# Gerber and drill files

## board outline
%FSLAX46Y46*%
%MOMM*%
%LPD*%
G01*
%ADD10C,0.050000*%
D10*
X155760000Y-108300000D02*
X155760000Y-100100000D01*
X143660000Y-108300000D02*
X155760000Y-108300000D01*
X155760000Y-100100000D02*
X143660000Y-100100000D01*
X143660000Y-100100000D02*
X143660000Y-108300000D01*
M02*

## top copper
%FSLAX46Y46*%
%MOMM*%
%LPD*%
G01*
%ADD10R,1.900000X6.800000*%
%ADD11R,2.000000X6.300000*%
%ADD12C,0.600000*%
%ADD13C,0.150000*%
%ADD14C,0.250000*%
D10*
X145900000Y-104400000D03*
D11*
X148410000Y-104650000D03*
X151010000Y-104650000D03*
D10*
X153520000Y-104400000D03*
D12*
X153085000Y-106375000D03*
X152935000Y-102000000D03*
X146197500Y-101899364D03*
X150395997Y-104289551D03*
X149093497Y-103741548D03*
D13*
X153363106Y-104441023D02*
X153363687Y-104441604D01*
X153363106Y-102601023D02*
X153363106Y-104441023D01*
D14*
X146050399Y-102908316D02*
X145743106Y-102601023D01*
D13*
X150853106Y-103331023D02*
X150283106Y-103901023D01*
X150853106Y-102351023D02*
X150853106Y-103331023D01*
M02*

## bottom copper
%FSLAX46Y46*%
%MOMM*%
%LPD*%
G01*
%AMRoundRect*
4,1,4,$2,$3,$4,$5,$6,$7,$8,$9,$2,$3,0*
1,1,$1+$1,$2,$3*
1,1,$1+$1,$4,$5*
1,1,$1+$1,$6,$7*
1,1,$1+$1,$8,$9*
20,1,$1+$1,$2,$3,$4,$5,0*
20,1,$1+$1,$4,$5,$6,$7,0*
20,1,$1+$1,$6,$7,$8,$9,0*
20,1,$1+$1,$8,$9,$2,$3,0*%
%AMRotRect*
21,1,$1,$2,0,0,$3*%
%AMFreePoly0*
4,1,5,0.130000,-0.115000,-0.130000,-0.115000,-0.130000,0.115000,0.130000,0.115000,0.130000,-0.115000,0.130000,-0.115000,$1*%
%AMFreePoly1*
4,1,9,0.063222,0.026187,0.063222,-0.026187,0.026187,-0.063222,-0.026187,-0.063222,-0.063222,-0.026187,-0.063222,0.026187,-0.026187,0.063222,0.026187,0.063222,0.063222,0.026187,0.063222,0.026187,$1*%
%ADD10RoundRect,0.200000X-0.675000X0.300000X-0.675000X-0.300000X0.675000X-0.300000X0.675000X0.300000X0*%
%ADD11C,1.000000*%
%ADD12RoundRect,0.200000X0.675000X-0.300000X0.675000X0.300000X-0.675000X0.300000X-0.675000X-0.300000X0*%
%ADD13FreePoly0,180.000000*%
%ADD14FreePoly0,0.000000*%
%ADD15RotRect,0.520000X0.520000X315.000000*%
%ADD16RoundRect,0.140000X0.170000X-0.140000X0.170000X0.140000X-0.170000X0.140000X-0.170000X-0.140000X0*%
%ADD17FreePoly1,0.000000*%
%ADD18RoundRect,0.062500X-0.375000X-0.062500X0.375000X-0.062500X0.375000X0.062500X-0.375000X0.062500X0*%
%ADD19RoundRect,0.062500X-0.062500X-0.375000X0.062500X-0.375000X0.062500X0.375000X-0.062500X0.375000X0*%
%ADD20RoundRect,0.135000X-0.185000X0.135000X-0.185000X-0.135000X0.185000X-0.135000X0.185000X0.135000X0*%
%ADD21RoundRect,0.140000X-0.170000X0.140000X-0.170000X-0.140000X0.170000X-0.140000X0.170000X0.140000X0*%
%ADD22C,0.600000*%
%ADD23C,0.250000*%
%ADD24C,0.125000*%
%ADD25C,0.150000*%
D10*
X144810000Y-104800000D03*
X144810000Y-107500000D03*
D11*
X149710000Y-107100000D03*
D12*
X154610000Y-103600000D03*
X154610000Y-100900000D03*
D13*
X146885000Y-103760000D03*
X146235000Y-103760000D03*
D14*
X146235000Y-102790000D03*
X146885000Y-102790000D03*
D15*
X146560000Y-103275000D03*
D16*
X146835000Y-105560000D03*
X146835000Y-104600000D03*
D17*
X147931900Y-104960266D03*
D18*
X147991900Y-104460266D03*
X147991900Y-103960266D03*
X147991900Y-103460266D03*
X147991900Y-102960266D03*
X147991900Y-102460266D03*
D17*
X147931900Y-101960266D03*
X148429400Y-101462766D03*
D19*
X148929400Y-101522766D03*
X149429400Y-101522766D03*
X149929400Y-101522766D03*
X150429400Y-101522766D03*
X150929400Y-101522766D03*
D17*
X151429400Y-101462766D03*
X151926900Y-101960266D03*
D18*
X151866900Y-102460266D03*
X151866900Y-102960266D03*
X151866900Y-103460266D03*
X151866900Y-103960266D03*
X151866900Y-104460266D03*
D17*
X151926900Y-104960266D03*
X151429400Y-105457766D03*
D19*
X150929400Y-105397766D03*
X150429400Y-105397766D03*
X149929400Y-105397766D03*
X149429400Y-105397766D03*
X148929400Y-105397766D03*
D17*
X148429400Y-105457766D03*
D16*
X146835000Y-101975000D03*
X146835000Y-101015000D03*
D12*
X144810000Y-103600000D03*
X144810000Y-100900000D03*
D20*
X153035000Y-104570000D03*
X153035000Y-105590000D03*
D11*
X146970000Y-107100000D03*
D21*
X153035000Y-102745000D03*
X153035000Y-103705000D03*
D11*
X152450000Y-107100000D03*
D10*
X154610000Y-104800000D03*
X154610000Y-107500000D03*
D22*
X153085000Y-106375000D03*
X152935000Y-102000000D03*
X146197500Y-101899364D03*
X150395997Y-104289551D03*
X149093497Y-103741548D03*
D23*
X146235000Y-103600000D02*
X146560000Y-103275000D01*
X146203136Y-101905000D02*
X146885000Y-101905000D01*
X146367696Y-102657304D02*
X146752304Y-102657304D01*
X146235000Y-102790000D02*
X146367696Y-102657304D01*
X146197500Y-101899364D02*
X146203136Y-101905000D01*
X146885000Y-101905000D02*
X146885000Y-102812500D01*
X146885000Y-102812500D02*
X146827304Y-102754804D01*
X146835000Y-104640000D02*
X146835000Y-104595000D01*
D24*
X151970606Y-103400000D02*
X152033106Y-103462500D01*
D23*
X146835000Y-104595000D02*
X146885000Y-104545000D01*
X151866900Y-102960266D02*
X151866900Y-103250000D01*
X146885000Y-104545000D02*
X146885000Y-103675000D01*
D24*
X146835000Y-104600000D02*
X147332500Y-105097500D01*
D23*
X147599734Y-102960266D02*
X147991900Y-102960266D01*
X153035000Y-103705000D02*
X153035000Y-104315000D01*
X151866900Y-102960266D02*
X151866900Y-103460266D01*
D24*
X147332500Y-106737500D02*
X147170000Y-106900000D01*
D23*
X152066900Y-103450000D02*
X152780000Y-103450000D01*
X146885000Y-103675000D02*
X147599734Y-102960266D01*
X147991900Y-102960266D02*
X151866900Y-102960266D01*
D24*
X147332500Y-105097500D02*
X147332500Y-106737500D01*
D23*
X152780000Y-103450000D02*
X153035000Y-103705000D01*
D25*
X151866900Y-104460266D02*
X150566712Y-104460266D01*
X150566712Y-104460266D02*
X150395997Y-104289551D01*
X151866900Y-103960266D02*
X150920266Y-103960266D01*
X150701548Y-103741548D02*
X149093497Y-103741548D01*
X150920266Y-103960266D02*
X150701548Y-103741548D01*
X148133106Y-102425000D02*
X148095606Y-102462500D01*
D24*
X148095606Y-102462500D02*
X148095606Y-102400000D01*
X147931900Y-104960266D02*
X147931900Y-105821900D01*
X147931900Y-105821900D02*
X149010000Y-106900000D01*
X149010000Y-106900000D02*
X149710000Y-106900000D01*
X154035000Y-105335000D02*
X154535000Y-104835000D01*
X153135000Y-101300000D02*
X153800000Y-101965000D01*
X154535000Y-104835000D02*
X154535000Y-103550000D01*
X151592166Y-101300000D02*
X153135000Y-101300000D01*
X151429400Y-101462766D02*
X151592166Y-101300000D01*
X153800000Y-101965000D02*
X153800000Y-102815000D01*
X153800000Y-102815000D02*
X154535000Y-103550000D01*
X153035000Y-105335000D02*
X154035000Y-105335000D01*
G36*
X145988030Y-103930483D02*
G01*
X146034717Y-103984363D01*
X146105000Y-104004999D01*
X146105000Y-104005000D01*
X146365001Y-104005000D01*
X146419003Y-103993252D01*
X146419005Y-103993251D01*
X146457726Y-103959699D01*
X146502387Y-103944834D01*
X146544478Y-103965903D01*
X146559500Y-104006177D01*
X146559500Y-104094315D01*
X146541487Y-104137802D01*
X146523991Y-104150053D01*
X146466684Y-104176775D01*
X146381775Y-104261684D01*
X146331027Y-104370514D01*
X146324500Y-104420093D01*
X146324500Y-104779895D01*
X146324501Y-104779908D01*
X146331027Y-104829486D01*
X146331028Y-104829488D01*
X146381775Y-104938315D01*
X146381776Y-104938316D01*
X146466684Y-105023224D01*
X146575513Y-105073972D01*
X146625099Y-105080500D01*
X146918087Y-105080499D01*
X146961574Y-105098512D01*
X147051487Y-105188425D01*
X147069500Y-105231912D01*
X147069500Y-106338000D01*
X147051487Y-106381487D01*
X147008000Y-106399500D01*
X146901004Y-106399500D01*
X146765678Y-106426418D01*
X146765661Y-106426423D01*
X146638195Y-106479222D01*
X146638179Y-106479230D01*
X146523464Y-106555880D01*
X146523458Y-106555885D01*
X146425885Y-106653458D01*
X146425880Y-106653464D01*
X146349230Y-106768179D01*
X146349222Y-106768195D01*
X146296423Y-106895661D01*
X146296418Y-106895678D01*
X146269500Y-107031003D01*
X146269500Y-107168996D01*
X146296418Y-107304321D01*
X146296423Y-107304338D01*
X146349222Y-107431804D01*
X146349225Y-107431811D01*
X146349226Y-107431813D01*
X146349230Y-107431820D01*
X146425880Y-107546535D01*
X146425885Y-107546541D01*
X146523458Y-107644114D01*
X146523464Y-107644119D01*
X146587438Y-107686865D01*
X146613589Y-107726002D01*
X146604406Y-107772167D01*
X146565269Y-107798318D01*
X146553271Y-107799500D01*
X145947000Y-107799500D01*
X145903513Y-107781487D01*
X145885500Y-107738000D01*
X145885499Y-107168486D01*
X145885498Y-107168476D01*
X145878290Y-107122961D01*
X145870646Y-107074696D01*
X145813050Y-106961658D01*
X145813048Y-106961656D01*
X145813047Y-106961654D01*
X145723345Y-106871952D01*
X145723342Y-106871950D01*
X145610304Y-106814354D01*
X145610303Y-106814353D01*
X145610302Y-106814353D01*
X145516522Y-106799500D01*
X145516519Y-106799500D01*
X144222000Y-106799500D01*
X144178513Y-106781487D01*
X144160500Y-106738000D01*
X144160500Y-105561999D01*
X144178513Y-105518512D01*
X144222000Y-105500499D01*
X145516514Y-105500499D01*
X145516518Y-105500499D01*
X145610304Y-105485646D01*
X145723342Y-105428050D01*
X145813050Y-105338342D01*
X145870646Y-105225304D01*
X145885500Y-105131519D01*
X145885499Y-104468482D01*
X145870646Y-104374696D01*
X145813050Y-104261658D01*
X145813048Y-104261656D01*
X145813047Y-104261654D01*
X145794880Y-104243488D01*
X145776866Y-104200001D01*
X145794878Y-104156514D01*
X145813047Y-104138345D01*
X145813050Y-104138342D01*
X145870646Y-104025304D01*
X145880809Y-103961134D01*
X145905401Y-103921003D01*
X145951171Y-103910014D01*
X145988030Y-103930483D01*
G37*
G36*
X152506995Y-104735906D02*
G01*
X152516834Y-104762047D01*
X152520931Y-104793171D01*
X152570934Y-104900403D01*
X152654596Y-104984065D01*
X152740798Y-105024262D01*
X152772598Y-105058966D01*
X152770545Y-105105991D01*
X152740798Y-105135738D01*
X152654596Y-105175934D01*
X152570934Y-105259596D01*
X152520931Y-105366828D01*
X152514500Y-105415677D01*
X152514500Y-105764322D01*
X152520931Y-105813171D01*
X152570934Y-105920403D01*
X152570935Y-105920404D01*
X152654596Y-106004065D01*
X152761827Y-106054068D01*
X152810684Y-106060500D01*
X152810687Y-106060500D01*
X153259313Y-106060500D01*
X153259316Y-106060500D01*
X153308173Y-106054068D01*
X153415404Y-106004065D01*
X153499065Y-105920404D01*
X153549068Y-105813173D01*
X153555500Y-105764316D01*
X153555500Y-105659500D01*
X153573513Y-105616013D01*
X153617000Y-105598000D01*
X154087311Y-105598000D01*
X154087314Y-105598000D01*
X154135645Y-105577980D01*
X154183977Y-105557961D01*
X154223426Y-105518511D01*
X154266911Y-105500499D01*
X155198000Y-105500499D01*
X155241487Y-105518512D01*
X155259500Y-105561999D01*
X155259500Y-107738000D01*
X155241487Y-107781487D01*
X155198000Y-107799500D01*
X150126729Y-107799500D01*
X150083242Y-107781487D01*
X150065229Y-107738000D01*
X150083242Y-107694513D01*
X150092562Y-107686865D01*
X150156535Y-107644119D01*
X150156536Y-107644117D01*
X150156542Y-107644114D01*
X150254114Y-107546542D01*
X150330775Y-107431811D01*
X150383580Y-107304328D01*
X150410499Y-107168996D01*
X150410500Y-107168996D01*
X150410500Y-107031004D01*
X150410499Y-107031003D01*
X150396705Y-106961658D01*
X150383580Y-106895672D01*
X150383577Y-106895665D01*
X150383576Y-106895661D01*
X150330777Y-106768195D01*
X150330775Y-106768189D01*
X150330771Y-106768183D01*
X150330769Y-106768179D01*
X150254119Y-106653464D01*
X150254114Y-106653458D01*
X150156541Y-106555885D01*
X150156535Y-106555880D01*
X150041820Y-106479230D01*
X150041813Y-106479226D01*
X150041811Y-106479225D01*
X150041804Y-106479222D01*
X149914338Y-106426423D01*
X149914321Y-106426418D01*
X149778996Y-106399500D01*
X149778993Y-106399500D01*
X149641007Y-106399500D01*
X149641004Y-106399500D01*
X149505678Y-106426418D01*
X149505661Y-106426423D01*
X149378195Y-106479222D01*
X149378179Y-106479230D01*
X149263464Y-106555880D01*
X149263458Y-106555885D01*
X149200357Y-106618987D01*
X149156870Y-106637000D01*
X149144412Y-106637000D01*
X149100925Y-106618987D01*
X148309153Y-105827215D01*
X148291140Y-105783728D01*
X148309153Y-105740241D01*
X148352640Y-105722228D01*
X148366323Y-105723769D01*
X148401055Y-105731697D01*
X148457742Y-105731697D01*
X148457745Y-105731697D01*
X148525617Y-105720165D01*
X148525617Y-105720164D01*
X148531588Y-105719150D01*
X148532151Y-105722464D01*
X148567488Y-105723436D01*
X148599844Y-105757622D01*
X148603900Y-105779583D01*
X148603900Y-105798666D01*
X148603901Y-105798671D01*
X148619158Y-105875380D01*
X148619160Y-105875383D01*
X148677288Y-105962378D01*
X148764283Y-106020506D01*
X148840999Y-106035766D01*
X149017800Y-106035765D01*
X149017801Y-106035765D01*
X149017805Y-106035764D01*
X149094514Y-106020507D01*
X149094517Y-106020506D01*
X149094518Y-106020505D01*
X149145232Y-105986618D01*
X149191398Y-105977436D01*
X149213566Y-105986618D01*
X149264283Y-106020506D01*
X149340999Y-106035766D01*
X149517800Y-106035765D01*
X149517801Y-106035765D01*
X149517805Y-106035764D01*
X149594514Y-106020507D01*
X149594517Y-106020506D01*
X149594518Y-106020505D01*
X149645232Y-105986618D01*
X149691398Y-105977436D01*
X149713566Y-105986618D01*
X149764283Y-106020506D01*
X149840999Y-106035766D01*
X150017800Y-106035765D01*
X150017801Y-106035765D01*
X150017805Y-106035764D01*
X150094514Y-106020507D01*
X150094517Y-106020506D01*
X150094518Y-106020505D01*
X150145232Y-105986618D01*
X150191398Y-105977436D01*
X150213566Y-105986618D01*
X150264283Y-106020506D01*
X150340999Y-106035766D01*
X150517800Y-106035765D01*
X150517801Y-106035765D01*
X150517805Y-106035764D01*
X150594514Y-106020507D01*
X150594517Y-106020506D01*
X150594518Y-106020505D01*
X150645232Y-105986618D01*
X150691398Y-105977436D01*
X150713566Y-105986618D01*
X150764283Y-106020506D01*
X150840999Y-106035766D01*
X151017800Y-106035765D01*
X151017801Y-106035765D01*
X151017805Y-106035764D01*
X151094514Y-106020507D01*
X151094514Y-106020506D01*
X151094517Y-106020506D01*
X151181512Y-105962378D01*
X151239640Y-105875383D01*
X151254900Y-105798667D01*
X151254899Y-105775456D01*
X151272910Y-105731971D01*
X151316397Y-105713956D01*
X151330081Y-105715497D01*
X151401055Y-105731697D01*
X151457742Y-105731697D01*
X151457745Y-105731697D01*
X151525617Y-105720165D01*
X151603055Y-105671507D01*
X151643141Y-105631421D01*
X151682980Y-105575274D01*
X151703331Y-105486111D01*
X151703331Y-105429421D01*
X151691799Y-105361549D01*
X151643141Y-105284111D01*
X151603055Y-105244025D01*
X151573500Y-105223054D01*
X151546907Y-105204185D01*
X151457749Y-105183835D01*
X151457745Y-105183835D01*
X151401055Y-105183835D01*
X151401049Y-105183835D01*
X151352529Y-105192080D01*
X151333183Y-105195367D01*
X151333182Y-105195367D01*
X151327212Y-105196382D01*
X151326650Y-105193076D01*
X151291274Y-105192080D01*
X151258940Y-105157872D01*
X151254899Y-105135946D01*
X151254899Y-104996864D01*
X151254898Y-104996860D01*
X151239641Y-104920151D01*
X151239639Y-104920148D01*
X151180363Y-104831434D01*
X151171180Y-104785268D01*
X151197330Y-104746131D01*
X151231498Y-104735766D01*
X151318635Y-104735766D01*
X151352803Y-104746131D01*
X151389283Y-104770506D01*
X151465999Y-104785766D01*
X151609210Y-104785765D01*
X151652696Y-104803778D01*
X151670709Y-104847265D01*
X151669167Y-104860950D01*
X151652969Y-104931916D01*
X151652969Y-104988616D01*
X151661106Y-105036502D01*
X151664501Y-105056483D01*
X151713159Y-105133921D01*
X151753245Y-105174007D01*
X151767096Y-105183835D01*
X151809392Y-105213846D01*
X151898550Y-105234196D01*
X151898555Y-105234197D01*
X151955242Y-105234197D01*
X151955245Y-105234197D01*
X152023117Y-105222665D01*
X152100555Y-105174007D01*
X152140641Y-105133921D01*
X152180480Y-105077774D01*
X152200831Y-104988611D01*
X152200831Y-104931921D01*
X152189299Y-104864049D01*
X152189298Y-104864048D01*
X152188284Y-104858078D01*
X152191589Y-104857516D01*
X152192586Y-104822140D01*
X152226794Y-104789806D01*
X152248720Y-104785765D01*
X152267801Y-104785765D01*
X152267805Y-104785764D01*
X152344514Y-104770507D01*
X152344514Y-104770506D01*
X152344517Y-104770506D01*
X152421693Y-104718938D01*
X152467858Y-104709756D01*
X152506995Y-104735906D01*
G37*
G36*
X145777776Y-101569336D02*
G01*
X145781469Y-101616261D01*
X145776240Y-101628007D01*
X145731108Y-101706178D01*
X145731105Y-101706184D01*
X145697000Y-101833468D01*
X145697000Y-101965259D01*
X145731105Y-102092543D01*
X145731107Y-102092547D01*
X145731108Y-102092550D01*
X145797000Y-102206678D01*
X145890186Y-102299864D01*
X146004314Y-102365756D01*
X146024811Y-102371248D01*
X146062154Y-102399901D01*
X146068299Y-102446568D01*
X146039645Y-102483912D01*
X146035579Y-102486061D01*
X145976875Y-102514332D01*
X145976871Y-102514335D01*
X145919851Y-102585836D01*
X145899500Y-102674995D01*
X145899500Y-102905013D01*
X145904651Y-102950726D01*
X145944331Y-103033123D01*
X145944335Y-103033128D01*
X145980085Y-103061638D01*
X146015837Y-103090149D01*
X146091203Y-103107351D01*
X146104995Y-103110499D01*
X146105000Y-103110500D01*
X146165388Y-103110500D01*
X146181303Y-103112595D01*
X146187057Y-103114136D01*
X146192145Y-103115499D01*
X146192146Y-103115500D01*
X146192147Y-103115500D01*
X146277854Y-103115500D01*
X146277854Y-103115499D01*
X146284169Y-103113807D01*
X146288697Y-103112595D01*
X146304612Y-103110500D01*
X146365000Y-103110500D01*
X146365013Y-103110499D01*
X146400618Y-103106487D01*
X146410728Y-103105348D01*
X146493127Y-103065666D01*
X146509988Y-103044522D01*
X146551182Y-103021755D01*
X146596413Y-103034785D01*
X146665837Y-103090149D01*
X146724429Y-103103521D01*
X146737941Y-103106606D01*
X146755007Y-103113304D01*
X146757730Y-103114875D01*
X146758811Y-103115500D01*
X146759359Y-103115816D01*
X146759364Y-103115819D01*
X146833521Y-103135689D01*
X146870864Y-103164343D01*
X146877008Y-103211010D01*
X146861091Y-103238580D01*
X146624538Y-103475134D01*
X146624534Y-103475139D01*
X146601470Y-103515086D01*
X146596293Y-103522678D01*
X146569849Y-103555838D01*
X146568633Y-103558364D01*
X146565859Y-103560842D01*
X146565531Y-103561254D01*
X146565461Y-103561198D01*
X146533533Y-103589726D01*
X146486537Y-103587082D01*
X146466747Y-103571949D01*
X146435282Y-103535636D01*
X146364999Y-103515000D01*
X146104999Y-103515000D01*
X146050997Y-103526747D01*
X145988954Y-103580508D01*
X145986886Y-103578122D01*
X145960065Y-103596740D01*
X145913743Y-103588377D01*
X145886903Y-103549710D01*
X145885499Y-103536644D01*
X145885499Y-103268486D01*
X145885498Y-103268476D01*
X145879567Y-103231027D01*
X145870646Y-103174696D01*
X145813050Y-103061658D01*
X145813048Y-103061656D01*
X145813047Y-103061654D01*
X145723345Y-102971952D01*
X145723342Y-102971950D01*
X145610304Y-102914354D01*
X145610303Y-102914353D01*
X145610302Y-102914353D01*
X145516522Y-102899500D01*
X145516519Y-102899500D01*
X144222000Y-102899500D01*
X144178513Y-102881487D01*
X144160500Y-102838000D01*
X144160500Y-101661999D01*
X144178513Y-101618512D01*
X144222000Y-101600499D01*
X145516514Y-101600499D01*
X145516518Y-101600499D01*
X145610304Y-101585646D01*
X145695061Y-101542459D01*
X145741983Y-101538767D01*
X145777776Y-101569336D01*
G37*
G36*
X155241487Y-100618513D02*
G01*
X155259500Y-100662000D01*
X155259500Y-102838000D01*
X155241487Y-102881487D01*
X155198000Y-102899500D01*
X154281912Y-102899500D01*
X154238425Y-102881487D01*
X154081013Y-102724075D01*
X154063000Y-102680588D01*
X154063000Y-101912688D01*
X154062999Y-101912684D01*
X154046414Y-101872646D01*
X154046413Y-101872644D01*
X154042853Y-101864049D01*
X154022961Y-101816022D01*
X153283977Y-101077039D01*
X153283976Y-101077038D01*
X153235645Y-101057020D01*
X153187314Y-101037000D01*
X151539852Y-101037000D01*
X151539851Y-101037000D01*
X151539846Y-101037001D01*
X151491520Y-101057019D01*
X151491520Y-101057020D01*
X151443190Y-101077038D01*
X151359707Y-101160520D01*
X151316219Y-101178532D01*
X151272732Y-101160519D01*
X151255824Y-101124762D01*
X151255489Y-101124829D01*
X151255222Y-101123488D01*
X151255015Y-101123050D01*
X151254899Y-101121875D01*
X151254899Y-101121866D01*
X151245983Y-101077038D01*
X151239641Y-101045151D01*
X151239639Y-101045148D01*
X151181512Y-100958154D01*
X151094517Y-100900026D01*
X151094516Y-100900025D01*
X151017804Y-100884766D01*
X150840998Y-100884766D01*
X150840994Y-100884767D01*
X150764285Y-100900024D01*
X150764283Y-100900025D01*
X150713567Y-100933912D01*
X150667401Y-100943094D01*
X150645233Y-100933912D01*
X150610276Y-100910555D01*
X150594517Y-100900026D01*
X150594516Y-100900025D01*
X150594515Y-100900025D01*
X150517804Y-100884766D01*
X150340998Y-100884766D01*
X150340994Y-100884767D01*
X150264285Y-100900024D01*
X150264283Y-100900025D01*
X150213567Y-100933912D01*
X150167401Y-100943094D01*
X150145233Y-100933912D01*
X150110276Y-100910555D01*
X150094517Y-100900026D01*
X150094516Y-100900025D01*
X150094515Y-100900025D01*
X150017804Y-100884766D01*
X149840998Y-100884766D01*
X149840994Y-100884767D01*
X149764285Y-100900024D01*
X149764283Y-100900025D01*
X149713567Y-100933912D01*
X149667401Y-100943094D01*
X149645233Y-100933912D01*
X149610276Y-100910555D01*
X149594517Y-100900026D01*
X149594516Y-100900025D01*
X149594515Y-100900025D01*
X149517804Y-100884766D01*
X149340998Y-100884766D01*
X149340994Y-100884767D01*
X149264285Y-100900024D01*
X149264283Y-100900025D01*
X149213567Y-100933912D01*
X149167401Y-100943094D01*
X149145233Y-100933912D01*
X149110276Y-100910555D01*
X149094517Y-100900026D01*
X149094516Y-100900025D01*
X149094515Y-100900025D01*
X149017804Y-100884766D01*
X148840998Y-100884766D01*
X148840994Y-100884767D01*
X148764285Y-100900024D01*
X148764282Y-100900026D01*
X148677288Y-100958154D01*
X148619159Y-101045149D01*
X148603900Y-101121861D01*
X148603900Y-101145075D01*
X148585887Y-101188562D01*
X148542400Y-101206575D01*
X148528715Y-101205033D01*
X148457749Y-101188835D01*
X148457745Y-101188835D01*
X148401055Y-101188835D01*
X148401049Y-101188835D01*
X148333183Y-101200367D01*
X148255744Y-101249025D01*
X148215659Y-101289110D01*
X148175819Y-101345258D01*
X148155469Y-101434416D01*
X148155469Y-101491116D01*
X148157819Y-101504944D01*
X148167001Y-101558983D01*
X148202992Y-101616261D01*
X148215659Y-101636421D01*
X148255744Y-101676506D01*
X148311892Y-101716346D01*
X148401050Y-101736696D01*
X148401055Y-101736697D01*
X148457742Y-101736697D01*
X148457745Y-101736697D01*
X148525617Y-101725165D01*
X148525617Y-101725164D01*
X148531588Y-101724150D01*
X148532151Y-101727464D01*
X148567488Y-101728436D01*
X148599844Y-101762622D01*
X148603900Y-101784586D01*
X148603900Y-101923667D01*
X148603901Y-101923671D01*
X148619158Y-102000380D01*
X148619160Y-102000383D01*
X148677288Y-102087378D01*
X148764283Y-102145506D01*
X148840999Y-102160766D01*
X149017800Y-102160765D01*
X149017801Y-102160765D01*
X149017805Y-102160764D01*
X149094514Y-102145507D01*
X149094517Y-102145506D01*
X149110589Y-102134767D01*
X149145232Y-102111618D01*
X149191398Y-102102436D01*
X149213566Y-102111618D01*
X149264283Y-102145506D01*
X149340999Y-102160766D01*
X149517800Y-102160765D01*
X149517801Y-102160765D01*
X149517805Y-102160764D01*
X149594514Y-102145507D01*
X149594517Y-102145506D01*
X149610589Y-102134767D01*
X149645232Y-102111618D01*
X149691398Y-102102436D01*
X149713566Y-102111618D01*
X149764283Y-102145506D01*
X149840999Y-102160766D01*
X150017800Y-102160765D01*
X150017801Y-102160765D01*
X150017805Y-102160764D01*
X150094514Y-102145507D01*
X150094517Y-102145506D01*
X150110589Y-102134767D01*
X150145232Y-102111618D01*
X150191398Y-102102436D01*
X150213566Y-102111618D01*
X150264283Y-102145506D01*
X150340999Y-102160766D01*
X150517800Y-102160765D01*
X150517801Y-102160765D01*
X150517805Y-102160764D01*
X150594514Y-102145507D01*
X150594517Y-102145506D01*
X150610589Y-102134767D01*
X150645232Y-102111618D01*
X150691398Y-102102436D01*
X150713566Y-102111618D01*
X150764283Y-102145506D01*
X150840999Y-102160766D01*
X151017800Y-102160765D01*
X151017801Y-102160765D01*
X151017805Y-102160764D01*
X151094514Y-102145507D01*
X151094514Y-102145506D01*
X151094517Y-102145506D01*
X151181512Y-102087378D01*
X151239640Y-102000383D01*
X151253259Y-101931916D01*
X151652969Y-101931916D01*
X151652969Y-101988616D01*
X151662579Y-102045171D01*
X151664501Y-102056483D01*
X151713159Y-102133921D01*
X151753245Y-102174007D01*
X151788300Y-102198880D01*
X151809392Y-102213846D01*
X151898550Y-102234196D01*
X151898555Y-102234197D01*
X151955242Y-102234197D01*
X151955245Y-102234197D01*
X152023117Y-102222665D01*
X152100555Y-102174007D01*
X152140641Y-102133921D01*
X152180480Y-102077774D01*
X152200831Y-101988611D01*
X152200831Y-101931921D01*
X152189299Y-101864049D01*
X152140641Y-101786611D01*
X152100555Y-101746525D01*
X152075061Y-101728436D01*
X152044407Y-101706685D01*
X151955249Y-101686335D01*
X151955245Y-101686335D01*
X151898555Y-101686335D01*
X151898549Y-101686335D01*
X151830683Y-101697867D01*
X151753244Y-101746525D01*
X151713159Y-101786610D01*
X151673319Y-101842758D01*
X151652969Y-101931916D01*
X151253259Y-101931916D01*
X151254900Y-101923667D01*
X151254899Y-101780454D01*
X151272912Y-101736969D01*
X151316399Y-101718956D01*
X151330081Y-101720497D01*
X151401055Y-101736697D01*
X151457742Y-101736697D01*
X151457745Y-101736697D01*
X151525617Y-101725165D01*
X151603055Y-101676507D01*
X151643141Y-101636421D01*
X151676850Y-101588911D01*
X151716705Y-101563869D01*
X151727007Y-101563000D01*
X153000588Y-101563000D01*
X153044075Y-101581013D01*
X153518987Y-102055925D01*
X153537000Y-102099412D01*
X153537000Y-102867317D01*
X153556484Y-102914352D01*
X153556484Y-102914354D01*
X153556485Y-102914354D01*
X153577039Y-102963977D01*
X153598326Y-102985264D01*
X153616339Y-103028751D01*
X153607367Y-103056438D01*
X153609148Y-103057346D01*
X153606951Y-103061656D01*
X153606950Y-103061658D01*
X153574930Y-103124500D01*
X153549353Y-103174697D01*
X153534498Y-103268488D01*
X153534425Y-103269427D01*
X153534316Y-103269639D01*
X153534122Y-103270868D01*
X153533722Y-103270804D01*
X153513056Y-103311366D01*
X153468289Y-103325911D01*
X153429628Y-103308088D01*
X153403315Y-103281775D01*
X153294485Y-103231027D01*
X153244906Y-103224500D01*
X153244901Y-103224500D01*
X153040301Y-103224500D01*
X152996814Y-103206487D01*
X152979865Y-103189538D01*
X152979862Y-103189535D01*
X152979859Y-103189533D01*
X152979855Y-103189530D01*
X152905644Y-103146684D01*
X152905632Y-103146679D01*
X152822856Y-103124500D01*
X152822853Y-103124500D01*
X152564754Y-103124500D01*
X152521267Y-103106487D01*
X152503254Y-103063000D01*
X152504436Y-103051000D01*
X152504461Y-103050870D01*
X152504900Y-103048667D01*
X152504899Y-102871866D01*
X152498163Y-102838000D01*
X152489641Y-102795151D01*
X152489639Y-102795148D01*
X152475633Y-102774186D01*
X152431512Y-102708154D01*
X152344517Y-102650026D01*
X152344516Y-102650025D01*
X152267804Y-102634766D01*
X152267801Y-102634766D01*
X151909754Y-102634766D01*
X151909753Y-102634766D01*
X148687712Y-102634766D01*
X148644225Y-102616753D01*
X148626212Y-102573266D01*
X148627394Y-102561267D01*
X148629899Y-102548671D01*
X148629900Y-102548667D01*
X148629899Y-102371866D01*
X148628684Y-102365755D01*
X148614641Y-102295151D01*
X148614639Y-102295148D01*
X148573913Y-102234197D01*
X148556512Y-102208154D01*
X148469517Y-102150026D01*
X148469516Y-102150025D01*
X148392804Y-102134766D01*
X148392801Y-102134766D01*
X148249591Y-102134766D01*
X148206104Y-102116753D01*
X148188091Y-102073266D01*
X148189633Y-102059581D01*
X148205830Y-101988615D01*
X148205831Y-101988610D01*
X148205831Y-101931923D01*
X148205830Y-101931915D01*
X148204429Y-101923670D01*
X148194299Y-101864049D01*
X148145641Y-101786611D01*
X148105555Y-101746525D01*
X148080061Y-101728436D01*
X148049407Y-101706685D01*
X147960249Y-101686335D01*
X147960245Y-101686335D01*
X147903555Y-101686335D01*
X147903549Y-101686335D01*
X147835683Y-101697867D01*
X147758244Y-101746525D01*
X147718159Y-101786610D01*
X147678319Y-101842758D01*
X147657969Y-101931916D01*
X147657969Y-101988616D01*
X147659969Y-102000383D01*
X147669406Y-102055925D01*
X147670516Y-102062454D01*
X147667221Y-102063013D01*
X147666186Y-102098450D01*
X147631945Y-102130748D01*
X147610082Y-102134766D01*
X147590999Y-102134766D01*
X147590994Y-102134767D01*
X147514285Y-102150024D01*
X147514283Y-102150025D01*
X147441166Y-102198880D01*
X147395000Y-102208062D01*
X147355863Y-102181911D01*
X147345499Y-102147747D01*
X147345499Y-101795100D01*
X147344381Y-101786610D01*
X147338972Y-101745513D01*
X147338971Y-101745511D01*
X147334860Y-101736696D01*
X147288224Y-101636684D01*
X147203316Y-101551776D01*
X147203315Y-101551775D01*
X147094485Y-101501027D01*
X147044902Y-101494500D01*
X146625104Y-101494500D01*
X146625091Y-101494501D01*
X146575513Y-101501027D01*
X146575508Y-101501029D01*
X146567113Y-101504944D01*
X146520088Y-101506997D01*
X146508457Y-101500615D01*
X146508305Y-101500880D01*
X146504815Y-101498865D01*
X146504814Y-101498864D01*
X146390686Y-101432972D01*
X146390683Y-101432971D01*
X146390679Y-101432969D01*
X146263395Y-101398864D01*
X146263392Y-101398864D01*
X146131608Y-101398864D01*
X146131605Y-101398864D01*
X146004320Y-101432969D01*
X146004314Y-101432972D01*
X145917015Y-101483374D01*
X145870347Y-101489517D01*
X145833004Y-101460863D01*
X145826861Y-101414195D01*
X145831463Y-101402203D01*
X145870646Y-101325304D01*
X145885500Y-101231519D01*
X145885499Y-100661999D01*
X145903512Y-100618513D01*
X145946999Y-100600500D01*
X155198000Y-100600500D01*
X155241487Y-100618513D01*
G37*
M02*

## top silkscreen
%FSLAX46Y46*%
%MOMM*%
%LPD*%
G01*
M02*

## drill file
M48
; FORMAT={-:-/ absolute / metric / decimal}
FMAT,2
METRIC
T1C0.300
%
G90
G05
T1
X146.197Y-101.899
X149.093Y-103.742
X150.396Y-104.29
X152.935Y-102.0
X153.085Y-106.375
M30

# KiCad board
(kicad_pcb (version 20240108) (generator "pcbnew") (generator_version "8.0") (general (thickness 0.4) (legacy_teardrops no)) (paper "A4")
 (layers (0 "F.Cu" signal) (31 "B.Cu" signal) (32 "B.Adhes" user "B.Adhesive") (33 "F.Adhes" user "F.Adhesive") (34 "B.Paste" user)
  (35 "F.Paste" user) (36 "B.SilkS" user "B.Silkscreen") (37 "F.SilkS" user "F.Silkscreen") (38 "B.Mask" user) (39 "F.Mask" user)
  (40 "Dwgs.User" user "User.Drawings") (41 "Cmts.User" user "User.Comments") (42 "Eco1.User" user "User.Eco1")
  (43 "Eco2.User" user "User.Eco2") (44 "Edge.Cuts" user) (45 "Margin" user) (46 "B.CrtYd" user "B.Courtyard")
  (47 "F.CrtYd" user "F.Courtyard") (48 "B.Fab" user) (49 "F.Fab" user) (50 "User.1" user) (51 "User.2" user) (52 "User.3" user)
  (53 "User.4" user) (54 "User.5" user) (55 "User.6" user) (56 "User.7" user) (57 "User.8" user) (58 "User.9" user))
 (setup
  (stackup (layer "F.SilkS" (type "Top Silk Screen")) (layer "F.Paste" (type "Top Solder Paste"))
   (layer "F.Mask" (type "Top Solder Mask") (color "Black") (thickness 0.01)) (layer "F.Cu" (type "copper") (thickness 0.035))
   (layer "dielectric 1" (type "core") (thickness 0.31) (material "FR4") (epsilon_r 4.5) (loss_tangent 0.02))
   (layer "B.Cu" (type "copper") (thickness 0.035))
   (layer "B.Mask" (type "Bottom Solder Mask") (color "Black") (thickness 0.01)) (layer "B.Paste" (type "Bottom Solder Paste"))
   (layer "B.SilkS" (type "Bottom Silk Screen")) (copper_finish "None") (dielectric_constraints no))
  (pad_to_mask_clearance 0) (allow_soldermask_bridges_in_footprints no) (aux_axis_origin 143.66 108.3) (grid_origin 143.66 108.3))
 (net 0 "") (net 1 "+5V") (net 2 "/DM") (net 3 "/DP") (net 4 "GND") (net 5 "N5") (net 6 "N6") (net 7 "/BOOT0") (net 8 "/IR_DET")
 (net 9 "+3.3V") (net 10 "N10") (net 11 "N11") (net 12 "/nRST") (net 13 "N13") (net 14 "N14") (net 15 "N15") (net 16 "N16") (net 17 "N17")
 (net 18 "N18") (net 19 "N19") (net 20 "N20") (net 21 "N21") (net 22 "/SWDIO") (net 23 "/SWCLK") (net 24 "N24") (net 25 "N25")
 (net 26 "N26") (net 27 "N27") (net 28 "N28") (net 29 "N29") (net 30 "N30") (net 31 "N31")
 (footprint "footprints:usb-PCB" (layer "F.Cu") (at 149.71 100.1 180)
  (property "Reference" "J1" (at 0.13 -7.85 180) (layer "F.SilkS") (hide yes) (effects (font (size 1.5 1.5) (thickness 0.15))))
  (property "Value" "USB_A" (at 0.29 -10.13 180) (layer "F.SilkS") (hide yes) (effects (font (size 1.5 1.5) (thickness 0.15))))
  (pad "1" connect rect (at 3.81 -4.3 180) (size 1.9 6.8) (layers "F.Cu" "F.Mask") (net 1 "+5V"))
  (pad "2" connect rect (at 1.3 -4.55 180) (size 2 6.3) (layers "F.Cu" "F.Mask") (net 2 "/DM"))
  (pad "3" connect rect (at -1.3 -4.55 180) (size 2 6.3) (layers "F.Cu" "F.Mask") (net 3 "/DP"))
  (pad "4" connect rect (at -3.81 -4.3 180) (size 1.9 6.8) (layers "F.Cu" "F.Mask") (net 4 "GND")))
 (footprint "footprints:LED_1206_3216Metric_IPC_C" (layer "B.Cu") (at 144.81 106.15 -90)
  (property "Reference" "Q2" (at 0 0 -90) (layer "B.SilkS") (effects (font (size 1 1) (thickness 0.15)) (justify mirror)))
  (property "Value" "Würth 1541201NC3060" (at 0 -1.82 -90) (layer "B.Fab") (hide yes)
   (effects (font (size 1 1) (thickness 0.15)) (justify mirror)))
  (pad "1" smd roundrect (at -1.35 0 270) (size 1 1.75) (layers "B.Cu" "B.Paste" "B.Mask") (roundrect_rratio 0.2) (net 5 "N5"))
  (pad "2" smd roundrect (at 1.35 0 270) (size 1 1.75) (layers "B.Cu" "B.Paste" "B.Mask") (roundrect_rratio 0.2) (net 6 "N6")))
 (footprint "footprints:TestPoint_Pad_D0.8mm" (layer "B.Cu") (at 150.01 106.55 180)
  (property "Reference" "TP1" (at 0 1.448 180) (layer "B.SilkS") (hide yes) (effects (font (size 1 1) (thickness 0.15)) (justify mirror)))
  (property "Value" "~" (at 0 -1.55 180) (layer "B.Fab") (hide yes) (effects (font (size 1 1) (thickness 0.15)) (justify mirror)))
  (pad "1" smd circle (at 0.3 -0.55 180) (size 1 1) (layers "B.Cu" "B.Mask") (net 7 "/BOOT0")))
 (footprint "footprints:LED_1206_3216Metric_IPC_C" (layer "B.Cu") (at 154.61 102.25 90)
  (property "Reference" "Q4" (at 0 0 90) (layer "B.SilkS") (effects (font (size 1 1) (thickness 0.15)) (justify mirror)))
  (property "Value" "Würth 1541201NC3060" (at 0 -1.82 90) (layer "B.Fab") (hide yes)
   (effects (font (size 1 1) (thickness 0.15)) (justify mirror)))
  (pad "1" smd roundrect (at -1.35 0 90) (size 1 1.75) (layers "B.Cu" "B.Paste" "B.Mask") (roundrect_rratio 0.2) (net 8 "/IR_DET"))
  (pad "2" smd roundrect (at 1.35 0 90) (size 1 1.75) (layers "B.Cu" "B.Paste" "B.Mask") (roundrect_rratio 0.2) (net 4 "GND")))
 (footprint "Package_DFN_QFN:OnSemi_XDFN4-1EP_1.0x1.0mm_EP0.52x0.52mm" (layer "B.Cu") (at 146.56 103.275 90)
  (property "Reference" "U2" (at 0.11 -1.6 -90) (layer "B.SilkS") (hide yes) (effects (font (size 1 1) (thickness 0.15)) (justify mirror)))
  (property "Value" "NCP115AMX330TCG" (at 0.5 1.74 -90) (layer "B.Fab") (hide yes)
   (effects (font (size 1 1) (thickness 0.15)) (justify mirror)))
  (pad "1" smd custom (at -0.485 0.325 180) (size 0.26 0.23) (layers "B.Cu" "B.Paste" "B.Mask") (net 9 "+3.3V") (zone_connect 0)
   (thermal_bridge_angle 45) (options (clearance outline) (anchor rect)) (primitives))
  (pad "2" smd custom (at -0.485 -0.325 180) (size 0.26 0.23) (layers "B.Cu" "B.Paste" "B.Mask") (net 4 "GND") (zone_connect 0)
   (thermal_bridge_angle 45) (options (clearance outline) (anchor rect)) (primitives))
  (pad "3" smd custom (at 0.485 -0.325) (size 0.26 0.23) (layers "B.Cu" "B.Paste" "B.Mask") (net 1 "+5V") (zone_connect 0)
   (thermal_bridge_angle 45) (options (clearance outline) (anchor rect)) (primitives))
  (pad "4" smd custom (at 0.485 0.325) (size 0.26 0.23) (layers "B.Cu" "B.Paste" "B.Mask") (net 1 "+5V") (zone_connect 0)
   (thermal_bridge_angle 45) (options (clearance outline) (anchor rect)) (primitives))
  (pad "5" smd rect (at 0 0 315) (size 0.52 0.52) (layers "B.Cu" "B.Paste" "B.Mask") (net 4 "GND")))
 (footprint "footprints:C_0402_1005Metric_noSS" (layer "B.Cu") (at 146.835 105.08 90)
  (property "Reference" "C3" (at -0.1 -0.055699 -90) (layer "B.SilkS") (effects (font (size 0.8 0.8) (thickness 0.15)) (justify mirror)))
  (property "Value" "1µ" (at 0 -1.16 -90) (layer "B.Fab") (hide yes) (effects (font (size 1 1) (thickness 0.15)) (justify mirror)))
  (pad "1" smd roundrect (at -0.48 0 90) (size 0.56 0.62) (layers "B.Cu" "B.Paste" "B.Mask") (roundrect_rratio 0.25) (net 4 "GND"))
  (pad "2" smd roundrect (at 0.48 0 90) (size 0.56 0.62) (layers "B.Cu" "B.Paste" "B.Mask") (roundrect_rratio 0.25) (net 9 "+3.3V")))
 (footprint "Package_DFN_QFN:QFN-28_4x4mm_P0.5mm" (layer "B.Cu") (at 149.9294 103.460266)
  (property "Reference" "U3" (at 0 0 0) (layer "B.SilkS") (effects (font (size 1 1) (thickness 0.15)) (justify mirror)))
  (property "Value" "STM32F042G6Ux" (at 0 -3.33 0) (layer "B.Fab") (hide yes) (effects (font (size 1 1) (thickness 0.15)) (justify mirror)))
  (pad "1" smd custom (at -1.9975 1.5) (size 0.136863 0.136863) (layers "B.Cu" "B.Paste" "B.Mask") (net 7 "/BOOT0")
   (options (clearance outline) (anchor circle)) (primitives))
  (pad "2" smd roundrect (at -1.9375 1) (size 0.875 0.25) (layers "B.Cu" "B.Paste" "B.Mask") (roundrect_rratio 0.25) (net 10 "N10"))
  (pad "3" smd roundrect (at -1.9375 0.5) (size 0.875 0.25) (layers "B.Cu" "B.Paste" "B.Mask") (roundrect_rratio 0.25) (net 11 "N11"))
  (pad "4" smd roundrect (at -1.9375 0) (size 0.875 0.25) (layers "B.Cu" "B.Paste" "B.Mask") (roundrect_rratio 0.25) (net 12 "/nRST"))
  (pad "5" smd roundrect (at -1.9375 -0.5) (size 0.875 0.25) (layers "B.Cu" "B.Paste" "B.Mask") (roundrect_rratio 0.25) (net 9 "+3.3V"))
  (pad "6" smd roundrect (at -1.9375 -1) (size 0.875 0.25) (layers "B.Cu" "B.Paste" "B.Mask") (roundrect_rratio 0.25) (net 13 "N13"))
  (pad "7" smd custom (at -1.9975 -1.5) (size 0.136863 0.136863) (layers "B.Cu" "B.Paste" "B.Mask") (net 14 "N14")
   (options (clearance outline) (anchor circle)) (primitives))
  (pad "8" smd custom (at -1.5 -1.9975) (size 0.136863 0.136863) (layers "B.Cu" "B.Paste" "B.Mask") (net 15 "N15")
   (options (clearance outline) (anchor circle)) (primitives))
  (pad "9" smd roundrect (at -1 -1.9375) (size 0.25 0.875) (layers "B.Cu" "B.Paste" "B.Mask") (roundrect_rratio 0.25) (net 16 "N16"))
  (pad "10" smd roundrect (at -0.5 -1.9375) (size 0.25 0.875) (layers "B.Cu" "B.Paste" "B.Mask") (roundrect_rratio 0.25) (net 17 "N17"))
  (pad "11" smd roundrect (at 0 -1.9375) (size 0.25 0.875) (layers "B.Cu" "B.Paste" "B.Mask") (roundrect_rratio 0.25) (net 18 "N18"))
  (pad "12" smd roundrect (at 0.5 -1.9375) (size 0.25 0.875) (layers "B.Cu" "B.Paste" "B.Mask") (roundrect_rratio 0.25) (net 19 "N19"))
  (pad "13" smd roundrect (at 1 -1.9375) (size 0.25 0.875) (layers "B.Cu" "B.Paste" "B.Mask") (roundrect_rratio 0.25) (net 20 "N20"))
  (pad "14" smd custom (at 1.5 -1.9975) (size 0.136863 0.136863) (layers "B.Cu" "B.Paste" "B.Mask") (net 8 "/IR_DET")
   (options (clearance outline) (anchor circle)) (primitives))
  (pad "15" smd custom (at 1.9975 -1.5) (size 0.136863 0.136863) (layers "B.Cu" "B.Paste" "B.Mask") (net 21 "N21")
   (options (clearance outline) (anchor circle)) (primitives))
  (pad "16" smd roundrect (at 1.9375 -1) (size 0.875 0.25) (layers "B.Cu" "B.Paste" "B.Mask") (roundrect_rratio 0.25) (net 4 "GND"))
  (pad "17" smd roundrect (at 1.9375 -0.5) (size 0.875 0.25) (layers "B.Cu" "B.Paste" "B.Mask") (roundrect_rratio 0.25) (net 9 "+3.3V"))
  (pad "18" smd roundrect (at 1.9375 0) (size 0.875 0.25) (layers "B.Cu" "B.Paste" "B.Mask") (roundrect_rratio 0.25) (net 9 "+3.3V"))
  (pad "19" smd roundrect (at 1.9375 0.5) (size 0.875 0.25) (layers "B.Cu" "B.Paste" "B.Mask") (roundrect_rratio 0.25) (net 2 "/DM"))
  (pad "20" smd roundrect (at 1.9375 1) (size 0.875 0.25) (layers "B.Cu" "B.Paste" "B.Mask") (roundrect_rratio 0.25) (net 3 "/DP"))
  (pad "21" smd custom (at 1.9975 1.5) (size 0.136863 0.136863) (layers "B.Cu" "B.Paste" "B.Mask") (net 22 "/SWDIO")
   (options (clearance outline) (anchor circle)) (primitives))
  (pad "22" smd custom (at 1.5 1.9975) (size 0.136863 0.136863) (layers "B.Cu" "B.Paste" "B.Mask") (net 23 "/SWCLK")
   (options (clearance outline) (anchor circle)) (primitives))
  (pad "23" smd roundrect (at 1 1.9375) (size 0.25 0.875) (layers "B.Cu" "B.Paste" "B.Mask") (roundrect_rratio 0.25) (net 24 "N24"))
  (pad "24" smd roundrect (at 0.5 1.9375) (size 0.25 0.875) (layers "B.Cu" "B.Paste" "B.Mask") (roundrect_rratio 0.25) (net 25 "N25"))
  (pad "25" smd roundrect (at 0 1.9375) (size 0.25 0.875) (layers "B.Cu" "B.Paste" "B.Mask") (roundrect_rratio 0.25) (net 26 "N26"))
  (pad "26" smd roundrect (at -0.5 1.9375) (size 0.25 0.875) (layers "B.Cu" "B.Paste" "B.Mask") (roundrect_rratio 0.25) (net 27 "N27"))
  (pad "27" smd roundrect (at -1 1.9375) (size 0.25 0.875) (layers "B.Cu" "B.Paste" "B.Mask") (roundrect_rratio 0.25) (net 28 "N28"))
  (pad "28" smd custom (at -1.5 1.9975) (size 0.136863 0.136863) (layers "B.Cu" "B.Paste" "B.Mask") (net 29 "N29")
   (options (clearance outline) (anchor circle)) (primitives)))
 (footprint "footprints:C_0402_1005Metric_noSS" (layer "B.Cu") (at 146.835 101.495 90)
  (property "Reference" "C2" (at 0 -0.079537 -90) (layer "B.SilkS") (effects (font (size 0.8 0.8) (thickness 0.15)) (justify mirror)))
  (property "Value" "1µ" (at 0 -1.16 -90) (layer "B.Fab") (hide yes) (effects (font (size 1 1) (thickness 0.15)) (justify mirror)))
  (pad "1" smd roundrect (at -0.48 0 90) (size 0.56 0.62) (layers "B.Cu" "B.Paste" "B.Mask") (roundrect_rratio 0.25) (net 1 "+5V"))
  (pad "2" smd roundrect (at 0.48 0 90) (size 0.56 0.62) (layers "B.Cu" "B.Paste" "B.Mask") (roundrect_rratio 0.25) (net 4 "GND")))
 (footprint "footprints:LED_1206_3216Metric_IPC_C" (layer "B.Cu") (at 144.81 102.25 90)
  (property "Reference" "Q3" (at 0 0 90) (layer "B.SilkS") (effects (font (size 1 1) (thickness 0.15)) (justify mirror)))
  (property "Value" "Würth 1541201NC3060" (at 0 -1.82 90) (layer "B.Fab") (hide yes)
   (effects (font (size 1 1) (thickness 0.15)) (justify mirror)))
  (pad "1" smd roundrect (at -1.35 0 90) (size 1 1.75) (layers "B.Cu" "B.Paste" "B.Mask") (roundrect_rratio 0.2) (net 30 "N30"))
  (pad "2" smd roundrect (at 1.35 0 90) (size 1 1.75) (layers "B.Cu" "B.Paste" "B.Mask") (roundrect_rratio 0.2) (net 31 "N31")))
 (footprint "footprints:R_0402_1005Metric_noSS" (layer "B.Cu") (at 153.035 105.08 -90)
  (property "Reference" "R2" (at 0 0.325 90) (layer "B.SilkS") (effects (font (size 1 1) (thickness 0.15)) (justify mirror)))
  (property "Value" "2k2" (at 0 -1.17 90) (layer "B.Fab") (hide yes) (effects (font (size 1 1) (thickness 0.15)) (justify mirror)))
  (pad "1" smd roundrect (at -0.51 0 270) (size 0.54 0.64) (layers "B.Cu" "B.Paste" "B.Mask") (roundrect_rratio 0.25) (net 9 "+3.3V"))
  (pad "2" smd roundrect (at 0.51 0 270) (size 0.54 0.64) (layers "B.Cu" "B.Paste" "B.Mask") (roundrect_rratio 0.25) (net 8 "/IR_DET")))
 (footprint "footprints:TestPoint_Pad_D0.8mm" (layer "B.Cu") (at 148.41 106.55)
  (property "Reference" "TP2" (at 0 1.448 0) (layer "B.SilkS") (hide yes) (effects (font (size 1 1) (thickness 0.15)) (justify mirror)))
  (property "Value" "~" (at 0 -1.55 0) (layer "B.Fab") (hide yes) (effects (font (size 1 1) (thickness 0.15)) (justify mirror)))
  (pad "1" smd circle (at -1.44 0.55) (size 1 0.8) (layers "B.Cu" "B.Mask") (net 9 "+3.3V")))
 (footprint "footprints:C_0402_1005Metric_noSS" (layer "B.Cu") (at 153.035 103.225 -90)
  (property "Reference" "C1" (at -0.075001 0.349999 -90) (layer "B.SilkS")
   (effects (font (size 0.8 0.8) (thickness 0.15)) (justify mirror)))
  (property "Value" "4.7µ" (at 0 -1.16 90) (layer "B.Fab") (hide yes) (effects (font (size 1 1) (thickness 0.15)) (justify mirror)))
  (pad "1" smd roundrect (at -0.48 0 270) (size 0.56 0.62) (layers "B.Cu" "B.Paste" "B.Mask") (roundrect_rratio 0.25) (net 4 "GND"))
  (pad "2" smd roundrect (at 0.48 0 270) (size 0.56 0.62) (layers "B.Cu" "B.Paste" "B.Mask") (roundrect_rratio 0.25) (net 9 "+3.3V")))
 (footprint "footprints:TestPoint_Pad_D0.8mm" (layer "B.Cu") (at 159.385 106.9 180)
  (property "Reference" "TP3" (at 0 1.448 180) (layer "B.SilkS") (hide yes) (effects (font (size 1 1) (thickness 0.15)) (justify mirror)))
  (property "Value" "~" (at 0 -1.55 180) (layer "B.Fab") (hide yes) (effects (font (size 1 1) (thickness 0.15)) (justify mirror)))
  (pad "1" smd circle (at 6.935 -0.2 180) (size 1 0.8) (layers "B.Cu" "B.Mask") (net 4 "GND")))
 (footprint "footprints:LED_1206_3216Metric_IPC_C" (layer "B.Cu") (at 154.61 106.15 -90)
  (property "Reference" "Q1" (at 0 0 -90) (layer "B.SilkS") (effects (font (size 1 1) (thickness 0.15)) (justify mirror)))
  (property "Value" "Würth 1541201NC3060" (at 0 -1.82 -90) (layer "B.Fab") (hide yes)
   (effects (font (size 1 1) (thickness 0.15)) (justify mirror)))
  (pad "1" smd roundrect (at -1.35 0 270) (size 1 1.75) (layers "B.Cu" "B.Paste" "B.Mask") (roundrect_rratio 0.2) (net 8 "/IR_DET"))
  (pad "2" smd roundrect (at 1.35 0 270) (size 1 1.75) (layers "B.Cu" "B.Paste" "B.Mask") (roundrect_rratio 0.2) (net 4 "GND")))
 (gr_line (start 155.76 108.3) (end 155.76 100.1) (stroke (width 0.05) (type default)) (layer "Edge.Cuts"))
 (gr_line (start 143.66 108.3) (end 155.76 108.3) (stroke (width 0.05) (type default)) (layer "Edge.Cuts"))
 (gr_line (start 155.76 100.1) (end 143.66 100.1) (stroke (width 0.05) (type default)) (layer "Edge.Cuts"))
 (gr_line (start 143.66 100.1) (end 143.66 108.3) (stroke (width 0.05) (type default)) (layer "Edge.Cuts"))
 (segment (start 153.363106 104.441023) (end 153.363687 104.441604) (width 0.15) (layer "F.Cu") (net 4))
 (segment (start 153.363106 102.601023) (end 153.363106 104.441023) (width 0.15) (layer "F.Cu") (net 4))
 (via (at 153.085 106.375) (size 0.6) (drill 0.3) (layers "F.Cu" "B.Cu") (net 4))
 (via (at 152.935 102) (size 0.6) (drill 0.3) (layers "F.Cu" "B.Cu") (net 4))
 (segment (start 146.235 103.6) (end 146.56 103.275) (width 0.25) (layer "B.Cu") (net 4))
 (segment (start 146.050399 102.908316) (end 145.743106 102.601023) (width 0.25) (layer "F.Cu") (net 1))
 (via (at 146.1975 101.899364) (size 0.6) (drill 0.3) (layers "F.Cu" "B.Cu") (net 1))
 (segment (start 146.203136 101.905) (end 146.885 101.905) (width 0.25) (layer "B.Cu") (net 1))
 (segment (start 146.367696 102.657304) (end 146.752304 102.657304) (width 0.25) (layer "B.Cu") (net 1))
 (segment (start 146.235 102.79) (end 146.367696 102.657304) (width 0.25) (layer "B.Cu") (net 1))
 (segment (start 146.1975 101.899364) (end 146.203136 101.905) (width 0.25) (layer "B.Cu") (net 1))
 (segment (start 146.885 101.905) (end 146.885 102.8125) (width 0.25) (layer "B.Cu") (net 1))
 (segment (start 146.885 102.8125) (end 146.827304 102.754804) (width 0.25) (layer "B.Cu") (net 1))
 (segment (start 146.835 104.64) (end 146.835 104.595) (width 0.25) (layer "B.Cu") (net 9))
 (segment (start 151.970606 103.4) (end 152.033106 103.4625) (width 0.125) (layer "B.Cu") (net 9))
 (segment (start 146.835 104.595) (end 146.885 104.545) (width 0.25) (layer "B.Cu") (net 9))
 (segment (start 151.8669 102.960266) (end 151.8669 103.25) (width 0.25) (layer "B.Cu") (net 9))
 (segment (start 146.885 104.545) (end 146.885 103.675) (width 0.25) (layer "B.Cu") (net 9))
 (segment (start 146.835 104.6) (end 147.3325 105.0975) (width 0.125) (layer "B.Cu") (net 9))
 (segment (start 147.599734 102.960266) (end 147.9919 102.960266) (width 0.25) (layer "B.Cu") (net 9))
 (segment (start 153.035 103.705) (end 153.035 104.315) (width 0.25) (layer "B.Cu") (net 9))
 (segment (start 151.8669 102.960266) (end 151.8669 103.460266) (width 0.25) (layer "B.Cu") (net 9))
 (segment (start 147.3325 106.7375) (end 147.17 106.9) (width 0.125) (layer "B.Cu") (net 9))
 (segment (start 152.0669 103.45) (end 152.78 103.45) (width 0.25) (layer "B.Cu") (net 9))
 (segment (start 146.885 103.675) (end 147.599734 102.960266) (width 0.25) (layer "B.Cu") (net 9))
 (segment (start 147.9919 102.960266) (end 151.8669 102.960266) (width 0.25) (layer "B.Cu") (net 9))
 (segment (start 147.3325 105.0975) (end 147.3325 106.7375) (width 0.125) (layer "B.Cu") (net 9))
 (segment (start 152.78 103.45) (end 153.035 103.705) (width 0.25) (layer "B.Cu") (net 9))
 (segment (start 150.853106 103.331023) (end 150.283106 103.901023) (width 0.15) (layer "F.Cu") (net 3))
 (segment (start 150.853106 102.351023) (end 150.853106 103.331023) (width 0.15) (layer "F.Cu") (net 3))
 (via (at 150.395997 104.289551) (size 0.6) (drill 0.3) (layers "F.Cu" "B.Cu") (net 3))
 (segment (start 151.8669 104.460266) (end 150.566712 104.460266) (width 0.15) (layer "B.Cu") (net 3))
 (segment (start 150.566712 104.460266) (end 150.395997 104.289551) (width 0.15) (layer "B.Cu") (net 3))
 (via (at 149.093497 103.741548) (size 0.6) (drill 0.3) (layers "F.Cu" "B.Cu") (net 2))
 (segment (start 151.8669 103.960266) (end 150.920266 103.960266) (width 0.15) (layer "B.Cu") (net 2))
 (segment (start 150.701548 103.741548) (end 149.093497 103.741548) (width 0.15) (layer "B.Cu") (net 2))
 (segment (start 150.920266 103.960266) (end 150.701548 103.741548) (width 0.15) (layer "B.Cu") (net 2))
 (segment (start 148.133106 102.425) (end 148.095606 102.4625) (width 0.15) (layer "B.Cu") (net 13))
 (segment (start 148.095606 102.4625) (end 148.095606 102.4) (width 0.125) (layer "B.Cu") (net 13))
 (segment (start 147.9319 104.960266) (end 147.9319 105.8219) (width 0.125) (layer "B.Cu") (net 7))
 (segment (start 147.9319 105.8219) (end 149.01 106.9) (width 0.125) (layer "B.Cu") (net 7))
 (segment (start 149.01 106.9) (end 149.71 106.9) (width 0.125) (layer "B.Cu") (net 7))
 (segment (start 154.035 105.335) (end 154.535 104.835) (width 0.125) (layer "B.Cu") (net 8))
 (segment (start 153.135 101.3) (end 153.8 101.965) (width 0.125) (layer "B.Cu") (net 8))
 (segment (start 154.535 104.835) (end 154.535 103.55) (width 0.125) (layer "B.Cu") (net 8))
 (segment (start 151.592166 101.3) (end 153.135 101.3) (width 0.125) (layer "B.Cu") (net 8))
 (segment (start 151.4294 101.462766) (end 151.592166 101.3) (width 0.125) (layer "B.Cu") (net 8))
 (segment (start 153.8 101.965) (end 153.8 102.815) (width 0.125) (layer "B.Cu") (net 8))
 (segment (start 153.8 102.815) (end 154.535 103.55) (width 0.125) (layer "B.Cu") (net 8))
 (segment (start 153.035 105.335) (end 154.035 105.335) (width 0.125) (layer "B.Cu") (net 8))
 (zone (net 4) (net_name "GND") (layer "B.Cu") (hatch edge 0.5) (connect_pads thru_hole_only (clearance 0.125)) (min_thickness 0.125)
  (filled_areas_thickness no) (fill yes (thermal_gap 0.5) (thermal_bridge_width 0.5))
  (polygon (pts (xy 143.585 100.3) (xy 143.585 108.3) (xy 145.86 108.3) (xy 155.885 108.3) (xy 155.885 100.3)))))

